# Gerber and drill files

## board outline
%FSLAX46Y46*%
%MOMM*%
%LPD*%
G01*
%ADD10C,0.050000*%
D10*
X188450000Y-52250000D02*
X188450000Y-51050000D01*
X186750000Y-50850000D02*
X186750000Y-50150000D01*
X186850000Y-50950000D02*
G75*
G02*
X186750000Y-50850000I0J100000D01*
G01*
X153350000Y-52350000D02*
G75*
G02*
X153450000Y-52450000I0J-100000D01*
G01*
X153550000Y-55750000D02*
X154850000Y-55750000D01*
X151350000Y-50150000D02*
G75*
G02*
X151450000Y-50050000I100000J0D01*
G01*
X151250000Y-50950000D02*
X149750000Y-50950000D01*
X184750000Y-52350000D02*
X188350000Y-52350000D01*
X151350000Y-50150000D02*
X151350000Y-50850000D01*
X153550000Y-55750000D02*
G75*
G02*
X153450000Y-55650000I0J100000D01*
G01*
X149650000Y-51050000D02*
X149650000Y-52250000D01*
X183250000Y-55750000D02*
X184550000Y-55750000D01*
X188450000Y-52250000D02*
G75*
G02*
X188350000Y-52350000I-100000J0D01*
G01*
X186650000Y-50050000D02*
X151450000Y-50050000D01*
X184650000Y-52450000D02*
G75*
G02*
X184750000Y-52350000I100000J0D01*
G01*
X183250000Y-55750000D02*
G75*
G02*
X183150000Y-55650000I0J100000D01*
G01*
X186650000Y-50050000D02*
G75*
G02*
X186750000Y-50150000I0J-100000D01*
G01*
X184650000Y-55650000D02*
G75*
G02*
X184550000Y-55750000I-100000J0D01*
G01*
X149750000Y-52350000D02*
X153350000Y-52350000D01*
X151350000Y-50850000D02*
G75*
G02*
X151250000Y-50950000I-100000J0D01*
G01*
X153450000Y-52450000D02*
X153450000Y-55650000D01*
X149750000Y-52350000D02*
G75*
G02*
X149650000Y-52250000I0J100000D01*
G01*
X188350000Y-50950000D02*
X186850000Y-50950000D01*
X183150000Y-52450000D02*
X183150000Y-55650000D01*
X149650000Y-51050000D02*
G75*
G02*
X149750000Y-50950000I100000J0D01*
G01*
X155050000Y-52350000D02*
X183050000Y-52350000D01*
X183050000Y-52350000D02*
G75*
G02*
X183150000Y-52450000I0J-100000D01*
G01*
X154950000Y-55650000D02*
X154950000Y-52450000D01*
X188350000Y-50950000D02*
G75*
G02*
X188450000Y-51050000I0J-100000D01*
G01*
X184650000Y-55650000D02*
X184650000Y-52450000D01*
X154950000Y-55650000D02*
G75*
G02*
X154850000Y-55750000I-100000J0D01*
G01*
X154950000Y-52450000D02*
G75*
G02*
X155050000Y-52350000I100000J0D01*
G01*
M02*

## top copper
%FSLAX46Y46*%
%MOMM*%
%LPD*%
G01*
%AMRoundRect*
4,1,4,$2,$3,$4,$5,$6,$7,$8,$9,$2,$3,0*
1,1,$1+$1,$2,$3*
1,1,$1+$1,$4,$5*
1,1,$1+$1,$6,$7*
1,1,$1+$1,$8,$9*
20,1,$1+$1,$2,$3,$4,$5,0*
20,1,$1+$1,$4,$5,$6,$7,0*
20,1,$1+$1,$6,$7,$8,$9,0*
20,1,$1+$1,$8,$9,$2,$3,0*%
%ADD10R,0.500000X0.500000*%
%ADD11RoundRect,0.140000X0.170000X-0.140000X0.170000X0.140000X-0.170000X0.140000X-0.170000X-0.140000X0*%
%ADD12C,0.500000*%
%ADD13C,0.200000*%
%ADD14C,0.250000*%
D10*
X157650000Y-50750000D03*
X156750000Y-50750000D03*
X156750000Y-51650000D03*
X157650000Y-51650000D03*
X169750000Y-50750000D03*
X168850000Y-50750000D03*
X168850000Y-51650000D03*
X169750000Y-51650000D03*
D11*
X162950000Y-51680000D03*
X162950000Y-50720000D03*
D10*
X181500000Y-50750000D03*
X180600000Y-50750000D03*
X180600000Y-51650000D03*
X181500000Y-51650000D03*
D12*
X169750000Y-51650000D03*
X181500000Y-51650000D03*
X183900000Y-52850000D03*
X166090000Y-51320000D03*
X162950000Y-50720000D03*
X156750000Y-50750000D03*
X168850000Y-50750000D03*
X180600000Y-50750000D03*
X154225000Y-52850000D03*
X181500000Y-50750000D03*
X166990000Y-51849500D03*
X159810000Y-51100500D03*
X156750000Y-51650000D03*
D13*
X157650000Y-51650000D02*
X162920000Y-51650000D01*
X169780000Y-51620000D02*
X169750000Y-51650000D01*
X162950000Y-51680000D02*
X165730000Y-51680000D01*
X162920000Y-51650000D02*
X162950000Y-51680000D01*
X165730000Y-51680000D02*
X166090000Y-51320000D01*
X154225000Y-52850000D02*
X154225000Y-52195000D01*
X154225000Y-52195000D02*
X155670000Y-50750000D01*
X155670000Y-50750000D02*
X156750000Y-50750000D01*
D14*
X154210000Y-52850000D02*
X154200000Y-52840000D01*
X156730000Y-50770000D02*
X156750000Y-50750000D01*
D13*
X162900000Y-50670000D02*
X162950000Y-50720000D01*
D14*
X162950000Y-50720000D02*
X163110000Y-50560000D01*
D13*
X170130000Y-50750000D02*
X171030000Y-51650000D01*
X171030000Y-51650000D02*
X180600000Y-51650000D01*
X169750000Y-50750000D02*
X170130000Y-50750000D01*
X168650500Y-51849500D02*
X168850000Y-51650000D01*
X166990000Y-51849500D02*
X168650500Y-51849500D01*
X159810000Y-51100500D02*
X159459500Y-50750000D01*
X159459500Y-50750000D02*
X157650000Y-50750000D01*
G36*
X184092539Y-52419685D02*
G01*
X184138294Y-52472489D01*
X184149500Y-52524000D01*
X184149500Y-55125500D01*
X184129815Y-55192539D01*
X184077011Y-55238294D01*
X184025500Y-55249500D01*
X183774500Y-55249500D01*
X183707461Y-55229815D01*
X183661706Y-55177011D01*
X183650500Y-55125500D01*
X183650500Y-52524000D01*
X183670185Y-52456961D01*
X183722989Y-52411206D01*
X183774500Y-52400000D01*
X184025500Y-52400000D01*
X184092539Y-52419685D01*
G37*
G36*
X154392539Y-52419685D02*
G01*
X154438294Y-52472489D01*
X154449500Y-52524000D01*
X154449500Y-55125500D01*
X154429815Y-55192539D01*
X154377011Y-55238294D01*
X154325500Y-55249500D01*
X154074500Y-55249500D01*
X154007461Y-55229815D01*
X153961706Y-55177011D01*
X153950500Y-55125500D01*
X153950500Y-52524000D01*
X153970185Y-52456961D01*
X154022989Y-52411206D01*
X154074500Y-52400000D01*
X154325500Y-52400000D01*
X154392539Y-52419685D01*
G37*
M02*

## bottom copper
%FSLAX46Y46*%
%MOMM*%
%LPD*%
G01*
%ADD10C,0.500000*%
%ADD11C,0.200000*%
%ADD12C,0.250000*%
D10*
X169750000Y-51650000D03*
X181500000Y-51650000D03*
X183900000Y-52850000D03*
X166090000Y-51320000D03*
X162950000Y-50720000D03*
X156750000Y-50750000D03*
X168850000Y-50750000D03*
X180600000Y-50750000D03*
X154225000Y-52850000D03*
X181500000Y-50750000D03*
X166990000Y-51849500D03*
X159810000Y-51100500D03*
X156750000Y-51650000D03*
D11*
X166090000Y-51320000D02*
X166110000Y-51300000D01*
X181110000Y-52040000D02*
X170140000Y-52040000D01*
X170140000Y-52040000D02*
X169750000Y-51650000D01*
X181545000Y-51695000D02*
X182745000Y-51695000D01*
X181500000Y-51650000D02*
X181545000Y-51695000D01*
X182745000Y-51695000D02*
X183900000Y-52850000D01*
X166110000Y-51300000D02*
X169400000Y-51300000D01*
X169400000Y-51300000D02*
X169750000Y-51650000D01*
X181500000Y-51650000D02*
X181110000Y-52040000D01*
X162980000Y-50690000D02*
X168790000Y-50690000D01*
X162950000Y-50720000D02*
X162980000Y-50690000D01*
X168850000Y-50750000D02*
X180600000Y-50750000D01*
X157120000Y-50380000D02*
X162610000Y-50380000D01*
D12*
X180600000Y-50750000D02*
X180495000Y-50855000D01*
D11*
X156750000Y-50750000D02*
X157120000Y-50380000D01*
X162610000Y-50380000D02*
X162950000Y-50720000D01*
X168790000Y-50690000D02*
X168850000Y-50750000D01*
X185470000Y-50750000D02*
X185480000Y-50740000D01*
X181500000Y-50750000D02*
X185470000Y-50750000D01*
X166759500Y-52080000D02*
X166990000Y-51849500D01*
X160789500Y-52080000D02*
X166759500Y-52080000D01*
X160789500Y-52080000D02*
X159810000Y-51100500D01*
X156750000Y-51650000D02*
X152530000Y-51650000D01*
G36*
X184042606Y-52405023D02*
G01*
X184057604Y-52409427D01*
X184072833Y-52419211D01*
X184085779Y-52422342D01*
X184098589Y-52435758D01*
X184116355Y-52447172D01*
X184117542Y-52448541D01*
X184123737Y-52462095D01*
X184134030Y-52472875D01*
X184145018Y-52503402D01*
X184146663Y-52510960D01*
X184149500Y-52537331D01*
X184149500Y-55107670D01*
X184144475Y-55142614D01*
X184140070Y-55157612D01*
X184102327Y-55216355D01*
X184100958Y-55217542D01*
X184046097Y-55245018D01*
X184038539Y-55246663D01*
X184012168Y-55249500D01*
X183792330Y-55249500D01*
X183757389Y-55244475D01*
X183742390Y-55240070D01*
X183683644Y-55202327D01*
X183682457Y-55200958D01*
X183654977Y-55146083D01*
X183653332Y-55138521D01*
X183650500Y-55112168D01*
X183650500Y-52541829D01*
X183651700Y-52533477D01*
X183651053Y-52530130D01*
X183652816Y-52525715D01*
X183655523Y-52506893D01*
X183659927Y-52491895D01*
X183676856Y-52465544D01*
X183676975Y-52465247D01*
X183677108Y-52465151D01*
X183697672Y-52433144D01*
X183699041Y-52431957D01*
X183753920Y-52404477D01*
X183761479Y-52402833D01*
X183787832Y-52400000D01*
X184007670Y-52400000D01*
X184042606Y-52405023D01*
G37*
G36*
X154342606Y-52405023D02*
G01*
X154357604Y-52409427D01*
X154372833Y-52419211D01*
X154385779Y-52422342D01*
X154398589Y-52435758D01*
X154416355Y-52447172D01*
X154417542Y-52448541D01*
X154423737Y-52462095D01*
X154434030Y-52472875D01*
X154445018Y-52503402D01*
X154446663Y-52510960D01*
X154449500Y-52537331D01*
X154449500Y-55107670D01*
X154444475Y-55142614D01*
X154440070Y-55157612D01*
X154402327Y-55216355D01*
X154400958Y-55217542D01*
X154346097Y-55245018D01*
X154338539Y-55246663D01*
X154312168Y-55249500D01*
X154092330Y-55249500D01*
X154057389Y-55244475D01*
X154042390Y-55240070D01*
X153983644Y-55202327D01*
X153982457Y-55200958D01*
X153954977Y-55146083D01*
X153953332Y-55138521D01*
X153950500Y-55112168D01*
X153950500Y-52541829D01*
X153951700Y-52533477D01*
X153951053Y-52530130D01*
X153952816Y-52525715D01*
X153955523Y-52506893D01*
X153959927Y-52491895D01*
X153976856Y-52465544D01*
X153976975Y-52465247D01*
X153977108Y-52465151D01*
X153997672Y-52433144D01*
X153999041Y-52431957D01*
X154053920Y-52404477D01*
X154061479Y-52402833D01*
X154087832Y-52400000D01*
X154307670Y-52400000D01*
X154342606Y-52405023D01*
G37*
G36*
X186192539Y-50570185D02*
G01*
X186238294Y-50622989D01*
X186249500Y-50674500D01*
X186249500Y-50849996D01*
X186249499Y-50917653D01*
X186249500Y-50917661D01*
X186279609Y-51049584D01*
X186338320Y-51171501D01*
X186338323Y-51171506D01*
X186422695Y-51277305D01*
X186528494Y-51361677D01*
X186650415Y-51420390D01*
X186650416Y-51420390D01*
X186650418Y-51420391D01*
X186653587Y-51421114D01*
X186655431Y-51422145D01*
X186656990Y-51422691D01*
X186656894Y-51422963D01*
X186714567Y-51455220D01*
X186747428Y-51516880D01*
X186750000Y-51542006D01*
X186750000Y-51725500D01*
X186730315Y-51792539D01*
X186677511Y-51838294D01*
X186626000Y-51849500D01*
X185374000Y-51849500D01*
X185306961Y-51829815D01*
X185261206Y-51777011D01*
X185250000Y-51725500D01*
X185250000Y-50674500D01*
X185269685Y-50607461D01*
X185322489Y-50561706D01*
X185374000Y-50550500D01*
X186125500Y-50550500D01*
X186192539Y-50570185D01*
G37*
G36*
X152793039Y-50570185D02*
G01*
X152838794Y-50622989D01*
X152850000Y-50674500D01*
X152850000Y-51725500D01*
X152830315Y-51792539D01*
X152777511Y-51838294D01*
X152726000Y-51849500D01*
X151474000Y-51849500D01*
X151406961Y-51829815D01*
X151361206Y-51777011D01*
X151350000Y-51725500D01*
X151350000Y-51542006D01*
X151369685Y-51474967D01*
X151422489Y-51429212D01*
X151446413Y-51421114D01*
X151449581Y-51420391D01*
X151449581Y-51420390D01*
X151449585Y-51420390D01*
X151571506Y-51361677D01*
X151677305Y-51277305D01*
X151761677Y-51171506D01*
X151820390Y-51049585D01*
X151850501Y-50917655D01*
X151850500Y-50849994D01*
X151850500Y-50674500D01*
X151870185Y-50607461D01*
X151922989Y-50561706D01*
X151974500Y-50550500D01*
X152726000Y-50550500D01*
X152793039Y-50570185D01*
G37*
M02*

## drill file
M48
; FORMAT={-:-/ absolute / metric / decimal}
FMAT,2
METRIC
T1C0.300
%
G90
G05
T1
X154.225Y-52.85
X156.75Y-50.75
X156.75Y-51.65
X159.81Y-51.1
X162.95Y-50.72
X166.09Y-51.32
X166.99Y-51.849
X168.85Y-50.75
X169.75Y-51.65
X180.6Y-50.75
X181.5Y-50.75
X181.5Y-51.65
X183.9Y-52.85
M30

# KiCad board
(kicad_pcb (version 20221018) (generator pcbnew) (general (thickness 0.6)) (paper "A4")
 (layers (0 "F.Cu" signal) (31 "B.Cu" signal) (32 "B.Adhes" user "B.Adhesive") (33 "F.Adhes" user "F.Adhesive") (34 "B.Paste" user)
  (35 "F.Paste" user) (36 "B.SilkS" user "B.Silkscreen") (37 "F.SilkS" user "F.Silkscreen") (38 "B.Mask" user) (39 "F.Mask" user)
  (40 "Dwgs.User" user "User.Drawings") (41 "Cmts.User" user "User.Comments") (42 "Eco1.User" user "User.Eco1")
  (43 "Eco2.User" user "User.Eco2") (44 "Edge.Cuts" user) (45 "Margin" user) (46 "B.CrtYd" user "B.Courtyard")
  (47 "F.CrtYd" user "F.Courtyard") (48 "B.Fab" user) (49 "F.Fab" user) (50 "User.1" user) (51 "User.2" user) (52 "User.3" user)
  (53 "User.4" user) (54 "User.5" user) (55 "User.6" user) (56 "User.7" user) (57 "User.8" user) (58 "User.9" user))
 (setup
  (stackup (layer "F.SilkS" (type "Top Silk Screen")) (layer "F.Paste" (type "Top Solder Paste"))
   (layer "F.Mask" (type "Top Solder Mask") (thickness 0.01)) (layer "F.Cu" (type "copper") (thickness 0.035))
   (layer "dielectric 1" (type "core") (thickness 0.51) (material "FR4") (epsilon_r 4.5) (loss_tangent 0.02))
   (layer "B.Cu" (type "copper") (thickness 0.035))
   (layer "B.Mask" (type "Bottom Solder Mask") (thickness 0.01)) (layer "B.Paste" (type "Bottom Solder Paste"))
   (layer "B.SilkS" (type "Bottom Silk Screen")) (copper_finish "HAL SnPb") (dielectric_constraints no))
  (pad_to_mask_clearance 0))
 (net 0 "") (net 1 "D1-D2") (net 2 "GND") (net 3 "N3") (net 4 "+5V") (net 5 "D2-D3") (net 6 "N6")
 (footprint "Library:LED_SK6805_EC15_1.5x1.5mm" (layer "F.Cu") (at 157.2 51.2 -90)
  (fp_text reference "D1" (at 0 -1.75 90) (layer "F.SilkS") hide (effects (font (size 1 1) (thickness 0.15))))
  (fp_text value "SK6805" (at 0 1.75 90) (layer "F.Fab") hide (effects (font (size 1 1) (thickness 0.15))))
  (pad "1" smd rect (at -0.45 -0.45 270) (size 0.5 0.5) (layers "F.Cu" "F.Paste" "F.Mask") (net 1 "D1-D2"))
  (pad "2" smd rect (at -0.45 0.45 270) (size 0.5 0.5) (layers "F.Cu" "F.Paste" "F.Mask") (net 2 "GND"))
  (pad "3" smd rect (at 0.45 0.45 270) (size 0.5 0.5) (layers "F.Cu" "F.Paste" "F.Mask") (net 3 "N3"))
  (pad "4" smd rect (at 0.45 -0.45 270) (size 0.5 0.5) (layers "F.Cu" "F.Paste" "F.Mask") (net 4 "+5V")))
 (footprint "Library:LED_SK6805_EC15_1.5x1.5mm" (layer "F.Cu") (at 169.3 51.2 -90)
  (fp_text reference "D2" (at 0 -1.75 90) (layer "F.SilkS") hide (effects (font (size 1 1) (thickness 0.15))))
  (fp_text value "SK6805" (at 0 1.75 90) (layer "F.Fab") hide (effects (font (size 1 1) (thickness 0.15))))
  (pad "1" smd rect (at -0.45 -0.45 270) (size 0.5 0.5) (layers "F.Cu" "F.Paste" "F.Mask") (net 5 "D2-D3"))
  (pad "2" smd rect (at -0.45 0.45 270) (size 0.5 0.5) (layers "F.Cu" "F.Paste" "F.Mask") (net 2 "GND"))
  (pad "3" smd rect (at 0.45 0.45 270) (size 0.5 0.5) (layers "F.Cu" "F.Paste" "F.Mask") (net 1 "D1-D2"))
  (pad "4" smd rect (at 0.45 -0.45 270) (size 0.5 0.5) (layers "F.Cu" "F.Paste" "F.Mask") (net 4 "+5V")))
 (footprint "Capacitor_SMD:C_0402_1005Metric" (layer "F.Cu") (at 162.95 51.2 90)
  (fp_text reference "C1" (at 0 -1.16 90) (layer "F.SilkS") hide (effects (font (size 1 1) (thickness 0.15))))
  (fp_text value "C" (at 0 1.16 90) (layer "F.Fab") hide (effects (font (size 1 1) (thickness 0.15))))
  (pad "1" smd roundrect (at -0.48 0 90) (size 0.56 0.62) (layers "F.Cu" "F.Paste" "F.Mask") (roundrect_rratio 0.25) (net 4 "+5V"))
  (pad "2" smd roundrect (at 0.48 0 90) (size 0.56 0.62) (layers "F.Cu" "F.Paste" "F.Mask") (roundrect_rratio 0.25) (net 2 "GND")))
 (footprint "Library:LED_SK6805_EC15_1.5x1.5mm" (layer "F.Cu") (at 181.05 51.2 -90)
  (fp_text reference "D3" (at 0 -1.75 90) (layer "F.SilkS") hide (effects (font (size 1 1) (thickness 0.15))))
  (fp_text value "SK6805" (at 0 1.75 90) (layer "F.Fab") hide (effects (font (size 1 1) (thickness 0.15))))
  (pad "1" smd rect (at -0.45 -0.45 270) (size 0.5 0.5) (layers "F.Cu" "F.Paste" "F.Mask") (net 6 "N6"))
  (pad "2" smd rect (at -0.45 0.45 270) (size 0.5 0.5) (layers "F.Cu" "F.Paste" "F.Mask") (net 2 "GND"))
  (pad "3" smd rect (at 0.45 0.45 270) (size 0.5 0.5) (layers "F.Cu" "F.Paste" "F.Mask") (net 5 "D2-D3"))
  (pad "4" smd rect (at 0.45 -0.45 270) (size 0.5 0.5) (layers "F.Cu" "F.Paste" "F.Mask") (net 4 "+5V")))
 (gr_line (start 188.45 52.25) (end 188.45 51.05) (stroke (width 0.05) (type default)) (layer "Edge.Cuts"))
 (gr_line (start 186.75 50.85) (end 186.75 50.15) (stroke (width 0.05) (type default)) (layer "Edge.Cuts"))
 (gr_arc (start 186.85 50.95) (mid 186.779289 50.920711) (end 186.75 50.85) (stroke (width 0.05) (type default)) (layer "Edge.Cuts"))
 (gr_arc (start 153.35 52.35) (mid 153.420711 52.379289) (end 153.45 52.45) (stroke (width 0.05) (type default)) (layer "Edge.Cuts"))
 (gr_line (start 153.55 55.75) (end 154.85 55.75) (stroke (width 0.05) (type default)) (layer "Edge.Cuts"))
 (gr_arc (start 151.35 50.15) (mid 151.379289 50.079289) (end 151.45 50.05) (stroke (width 0.05) (type default)) (layer "Edge.Cuts"))
 (gr_line (start 151.25 50.95) (end 149.75 50.95) (stroke (width 0.05) (type default)) (layer "Edge.Cuts"))
 (gr_line (start 184.75 52.35) (end 188.35 52.35) (stroke (width 0.05) (type default)) (layer "Edge.Cuts"))
 (gr_line (start 151.35 50.15) (end 151.35 50.85) (stroke (width 0.05) (type default)) (layer "Edge.Cuts"))
 (gr_arc (start 153.55 55.75) (mid 153.479289 55.720711) (end 153.45 55.65) (stroke (width 0.05) (type default)) (layer "Edge.Cuts"))
 (gr_line (start 149.65 51.05) (end 149.65 52.25) (stroke (width 0.05) (type default)) (layer "Edge.Cuts"))
 (gr_line (start 183.25 55.75) (end 184.55 55.75) (stroke (width 0.05) (type default)) (layer "Edge.Cuts"))
 (gr_arc (start 188.45 52.25) (mid 188.420711 52.320711) (end 188.35 52.35) (stroke (width 0.05) (type default)) (layer "Edge.Cuts"))
 (gr_line (start 186.65 50.05) (end 151.45 50.05) (stroke (width 0.05) (type default)) (layer "Edge.Cuts"))
 (gr_arc (start 184.65 52.45) (mid 184.679289 52.379289) (end 184.75 52.35) (stroke (width 0.05) (type default)) (layer "Edge.Cuts"))
 (gr_arc (start 183.25 55.75) (mid 183.179289 55.720711) (end 183.15 55.65) (stroke (width 0.05) (type default)) (layer "Edge.Cuts"))
 (gr_arc (start 186.65 50.05) (mid 186.720711 50.079289) (end 186.75 50.15) (stroke (width 0.05) (type default)) (layer "Edge.Cuts"))
 (gr_arc (start 184.65 55.65) (mid 184.620711 55.720711) (end 184.55 55.75) (stroke (width 0.05) (type default)) (layer "Edge.Cuts"))
 (gr_line (start 149.75 52.35) (end 153.35 52.35) (stroke (width 0.05) (type default)) (layer "Edge.Cuts"))
 (gr_arc (start 151.35 50.85) (mid 151.320711 50.920711) (end 151.25 50.95) (stroke (width 0.05) (type default)) (layer "Edge.Cuts"))
 (gr_line (start 153.45 52.45) (end 153.45 55.65) (stroke (width 0.05) (type default)) (layer "Edge.Cuts"))
 (gr_arc (start 149.75 52.35) (mid 149.679289 52.320711) (end 149.65 52.25) (stroke (width 0.05) (type default)) (layer "Edge.Cuts"))
 (gr_line (start 188.35 50.95) (end 186.85 50.95) (stroke (width 0.05) (type default)) (layer "Edge.Cuts"))
 (gr_line (start 183.15 52.45) (end 183.15 55.65) (stroke (width 0.05) (type default)) (layer "Edge.Cuts"))
 (gr_arc (start 149.65 51.05) (mid 149.679289 50.979289) (end 149.75 50.95) (stroke (width 0.05) (type default)) (layer "Edge.Cuts"))
 (gr_line (start 155.05 52.35) (end 183.05 52.35) (stroke (width 0.05) (type default)) (layer "Edge.Cuts"))
 (gr_arc (start 183.05 52.35) (mid 183.120711 52.379289) (end 183.15 52.45) (stroke (width 0.05) (type default)) (layer "Edge.Cuts"))
 (gr_line (start 154.95 55.65) (end 154.95 52.45) (stroke (width 0.05) (type default)) (layer "Edge.Cuts"))
 (gr_arc (start 188.35 50.95) (mid 188.420711 50.979289) (end 188.45 51.05) (stroke (width 0.05) (type default)) (layer "Edge.Cuts"))
 (gr_line (start 184.65 55.65) (end 184.65 52.45) (stroke (width 0.05) (type default)) (layer "Edge.Cuts"))
 (gr_arc (start 154.95 55.65) (mid 154.920711 55.720711) (end 154.85 55.75) (stroke (width 0.05) (type default)) (layer "Edge.Cuts"))
 (gr_arc (start 154.95 52.45) (mid 154.979289 52.379289) (end 155.05 52.35) (stroke (width 0.05) (type default)) (layer "Edge.Cuts"))
 (segment (start 157.65 51.65) (end 162.92 51.65) (width 0.2) (layer "F.Cu") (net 4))
 (segment (start 169.78 51.62) (end 169.75 51.65) (width 0.2) (layer "F.Cu") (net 4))
 (segment (start 162.95 51.68) (end 165.73 51.68) (width 0.2) (layer "F.Cu") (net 4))
 (segment (start 162.92 51.65) (end 162.95 51.68) (width 0.2) (layer "F.Cu") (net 4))
 (segment (start 165.73 51.68) (end 166.09 51.32) (width 0.2) (layer "F.Cu") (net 4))
 (via (at 169.75 51.65) (size 0.5) (drill 0.3) (layers "F.Cu" "B.Cu") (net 4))
 (via (at 181.5 51.65) (size 0.5) (drill 0.3) (layers "F.Cu" "B.Cu") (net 4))
 (via (at 183.9 52.85) (size 0.5) (drill 0.3) (layers "F.Cu" "B.Cu") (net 4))
 (via (at 166.09 51.32) (size 0.5) (drill 0.3) (layers "F.Cu" "B.Cu") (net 4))
 (segment (start 166.09 51.32) (end 166.11 51.3) (width 0.2) (layer "B.Cu") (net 4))
 (segment (start 181.11 52.04) (end 170.14 52.04) (width 0.2) (layer "B.Cu") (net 4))
 (segment (start 170.14 52.04) (end 169.75 51.65) (width 0.2) (layer "B.Cu") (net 4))
 (segment (start 181.545 51.695) (end 182.745 51.695) (width 0.2) (layer "B.Cu") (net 4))
 (segment (start 181.5 51.65) (end 181.545 51.695) (width 0.2) (layer "B.Cu") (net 4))
 (segment (start 182.745 51.695) (end 183.9 52.85) (width 0.2) (layer "B.Cu") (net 4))
 (segment (start 166.11 51.3) (end 169.4 51.3) (width 0.2) (layer "B.Cu") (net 4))
 (segment (start 169.4 51.3) (end 169.75 51.65) (width 0.2) (layer "B.Cu") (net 4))
 (segment (start 181.5 51.65) (end 181.11 52.04) (width 0.2) (layer "B.Cu") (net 4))
 (segment (start 154.225 52.85) (end 154.225 52.195) (width 0.2) (layer "F.Cu") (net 2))
 (segment (start 154.225 52.195) (end 155.67 50.75) (width 0.2) (layer "F.Cu") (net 2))
 (segment (start 155.67 50.75) (end 156.75 50.75) (width 0.2) (layer "F.Cu") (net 2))
 (segment (start 154.21 52.85) (end 154.2 52.84) (width 0.25) (layer "F.Cu") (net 2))
 (segment (start 156.73 50.77) (end 156.75 50.75) (width 0.25) (layer "F.Cu") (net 2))
 (segment (start 162.9 50.67) (end 162.95 50.72) (width 0.2) (layer "F.Cu") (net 2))
 (segment (start 162.95 50.72) (end 163.11 50.56) (width 0.25) (layer "F.Cu") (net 2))
 (via (at 162.95 50.72) (size 0.5) (drill 0.3) (layers "F.Cu" "B.Cu") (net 2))
 (via (at 156.75 50.75) (size 0.5) (drill 0.3) (layers "F.Cu" "B.Cu") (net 2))
 (via (at 168.85 50.75) (size 0.5) (drill 0.3) (layers "F.Cu" "B.Cu") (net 2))
 (via (at 180.6 50.75) (size 0.5) (drill 0.3) (layers "F.Cu" "B.Cu") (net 2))
 (via (at 154.225 52.85) (size 0.5) (drill 0.3) (layers "F.Cu" "B.Cu") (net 2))
 (segment (start 162.98 50.69) (end 168.79 50.69) (width 0.2) (layer "B.Cu") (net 2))
 (segment (start 162.95 50.72) (end 162.98 50.69) (width 0.2) (layer "B.Cu") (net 2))
 (segment (start 168.85 50.75) (end 180.6 50.75) (width 0.2) (layer "B.Cu") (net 2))
 (segment (start 157.12 50.38) (end 162.61 50.38) (width 0.2) (layer "B.Cu") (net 2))
 (segment (start 180.6 50.75) (end 180.495 50.855) (width 0.25) (layer "B.Cu") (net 2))
 (segment (start 156.75 50.75) (end 157.12 50.38) (width 0.2) (layer "B.Cu") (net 2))
 (segment (start 162.61 50.38) (end 162.95 50.72) (width 0.2) (layer "B.Cu") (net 2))
 (segment (start 168.79 50.69) (end 168.85 50.75) (width 0.2) (layer "B.Cu") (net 2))
 (via (at 181.5 50.75) (size 0.5) (drill 0.3) (layers "F.Cu" "B.Cu") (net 6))
 (segment (start 185.47 50.75) (end 185.48 50.74) (width 0.2) (layer "B.Cu") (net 6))
 (segment (start 181.5 50.75) (end 185.47 50.75) (width 0.2) (layer "B.Cu") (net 6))
 (segment (start 170.13 50.75) (end 171.03 51.65) (width 0.2) (layer "F.Cu") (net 5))
 (segment (start 171.03 51.65) (end 180.6 51.65) (width 0.2) (layer "F.Cu") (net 5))
 (segment (start 169.75 50.75) (end 170.13 50.75) (width 0.2) (layer "F.Cu") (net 5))
 (segment (start 168.6505 51.8495) (end 168.85 51.65) (width 0.2) (layer "F.Cu") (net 1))
 (segment (start 166.99 51.8495) (end 168.6505 51.8495) (width 0.2) (layer "F.Cu") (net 1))
 (segment (start 159.81 51.1005) (end 159.4595 50.75) (width 0.2) (layer "F.Cu") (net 1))
 (segment (start 159.4595 50.75) (end 157.65 50.75) (width 0.2) (layer "F.Cu") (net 1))
 (via (at 166.99 51.8495) (size 0.5) (drill 0.3) (layers "F.Cu" "B.Cu") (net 1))
 (via (at 159.81 51.1005) (size 0.5) (drill 0.3) (layers "F.Cu" "B.Cu") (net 1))
 (segment (start 166.7595 52.08) (end 166.99 51.8495) (width 0.2) (layer "B.Cu") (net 1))
 (segment (start 160.7895 52.08) (end 166.7595 52.08) (width 0.2) (layer "B.Cu") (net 1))
 (segment (start 160.7895 52.08) (end 159.81 51.1005) (width 0.2) (layer "B.Cu") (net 1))
 (via (at 156.75 51.65) (size 0.5) (drill 0.3) (layers "F.Cu" "B.Cu") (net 3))
 (segment (start 156.75 51.65) (end 152.53 51.65) (width 0.2) (layer "B.Cu") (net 3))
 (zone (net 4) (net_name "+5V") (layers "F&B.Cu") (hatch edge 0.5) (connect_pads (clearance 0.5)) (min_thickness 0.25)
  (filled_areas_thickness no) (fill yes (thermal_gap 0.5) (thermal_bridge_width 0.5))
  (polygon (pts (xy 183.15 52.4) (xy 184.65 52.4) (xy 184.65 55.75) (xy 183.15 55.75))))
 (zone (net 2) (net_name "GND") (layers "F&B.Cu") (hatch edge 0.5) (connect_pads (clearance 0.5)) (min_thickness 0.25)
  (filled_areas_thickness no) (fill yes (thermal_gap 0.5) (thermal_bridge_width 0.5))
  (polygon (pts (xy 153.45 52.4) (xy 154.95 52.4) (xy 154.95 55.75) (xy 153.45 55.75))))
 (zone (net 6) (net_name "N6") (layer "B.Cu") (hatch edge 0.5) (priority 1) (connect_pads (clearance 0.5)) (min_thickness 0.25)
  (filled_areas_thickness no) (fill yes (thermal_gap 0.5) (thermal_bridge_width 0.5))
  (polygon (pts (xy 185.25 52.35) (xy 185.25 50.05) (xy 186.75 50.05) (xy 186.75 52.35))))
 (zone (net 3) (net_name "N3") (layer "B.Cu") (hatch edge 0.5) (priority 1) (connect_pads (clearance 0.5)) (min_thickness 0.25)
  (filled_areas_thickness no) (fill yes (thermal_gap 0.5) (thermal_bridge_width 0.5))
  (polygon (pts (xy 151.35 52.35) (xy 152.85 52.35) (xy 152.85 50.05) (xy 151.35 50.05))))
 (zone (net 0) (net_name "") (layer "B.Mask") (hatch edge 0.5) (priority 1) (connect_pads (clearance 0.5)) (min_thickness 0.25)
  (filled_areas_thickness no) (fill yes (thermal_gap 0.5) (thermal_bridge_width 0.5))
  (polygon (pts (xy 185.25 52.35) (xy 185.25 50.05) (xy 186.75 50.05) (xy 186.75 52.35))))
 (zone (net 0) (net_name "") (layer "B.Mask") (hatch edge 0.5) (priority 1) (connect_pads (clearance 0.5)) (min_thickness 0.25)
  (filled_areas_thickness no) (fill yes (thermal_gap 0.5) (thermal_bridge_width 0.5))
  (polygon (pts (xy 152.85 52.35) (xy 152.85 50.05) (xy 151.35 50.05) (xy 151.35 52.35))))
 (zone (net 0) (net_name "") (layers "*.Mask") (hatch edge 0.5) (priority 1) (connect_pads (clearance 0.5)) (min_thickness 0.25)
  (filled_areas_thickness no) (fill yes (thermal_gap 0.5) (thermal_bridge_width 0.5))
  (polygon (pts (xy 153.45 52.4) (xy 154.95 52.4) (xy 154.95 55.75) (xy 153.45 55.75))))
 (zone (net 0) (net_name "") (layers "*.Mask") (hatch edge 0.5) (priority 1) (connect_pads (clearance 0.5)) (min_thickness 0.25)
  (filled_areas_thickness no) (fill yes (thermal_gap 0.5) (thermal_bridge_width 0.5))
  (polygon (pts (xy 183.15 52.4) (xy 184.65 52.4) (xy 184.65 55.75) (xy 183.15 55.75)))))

